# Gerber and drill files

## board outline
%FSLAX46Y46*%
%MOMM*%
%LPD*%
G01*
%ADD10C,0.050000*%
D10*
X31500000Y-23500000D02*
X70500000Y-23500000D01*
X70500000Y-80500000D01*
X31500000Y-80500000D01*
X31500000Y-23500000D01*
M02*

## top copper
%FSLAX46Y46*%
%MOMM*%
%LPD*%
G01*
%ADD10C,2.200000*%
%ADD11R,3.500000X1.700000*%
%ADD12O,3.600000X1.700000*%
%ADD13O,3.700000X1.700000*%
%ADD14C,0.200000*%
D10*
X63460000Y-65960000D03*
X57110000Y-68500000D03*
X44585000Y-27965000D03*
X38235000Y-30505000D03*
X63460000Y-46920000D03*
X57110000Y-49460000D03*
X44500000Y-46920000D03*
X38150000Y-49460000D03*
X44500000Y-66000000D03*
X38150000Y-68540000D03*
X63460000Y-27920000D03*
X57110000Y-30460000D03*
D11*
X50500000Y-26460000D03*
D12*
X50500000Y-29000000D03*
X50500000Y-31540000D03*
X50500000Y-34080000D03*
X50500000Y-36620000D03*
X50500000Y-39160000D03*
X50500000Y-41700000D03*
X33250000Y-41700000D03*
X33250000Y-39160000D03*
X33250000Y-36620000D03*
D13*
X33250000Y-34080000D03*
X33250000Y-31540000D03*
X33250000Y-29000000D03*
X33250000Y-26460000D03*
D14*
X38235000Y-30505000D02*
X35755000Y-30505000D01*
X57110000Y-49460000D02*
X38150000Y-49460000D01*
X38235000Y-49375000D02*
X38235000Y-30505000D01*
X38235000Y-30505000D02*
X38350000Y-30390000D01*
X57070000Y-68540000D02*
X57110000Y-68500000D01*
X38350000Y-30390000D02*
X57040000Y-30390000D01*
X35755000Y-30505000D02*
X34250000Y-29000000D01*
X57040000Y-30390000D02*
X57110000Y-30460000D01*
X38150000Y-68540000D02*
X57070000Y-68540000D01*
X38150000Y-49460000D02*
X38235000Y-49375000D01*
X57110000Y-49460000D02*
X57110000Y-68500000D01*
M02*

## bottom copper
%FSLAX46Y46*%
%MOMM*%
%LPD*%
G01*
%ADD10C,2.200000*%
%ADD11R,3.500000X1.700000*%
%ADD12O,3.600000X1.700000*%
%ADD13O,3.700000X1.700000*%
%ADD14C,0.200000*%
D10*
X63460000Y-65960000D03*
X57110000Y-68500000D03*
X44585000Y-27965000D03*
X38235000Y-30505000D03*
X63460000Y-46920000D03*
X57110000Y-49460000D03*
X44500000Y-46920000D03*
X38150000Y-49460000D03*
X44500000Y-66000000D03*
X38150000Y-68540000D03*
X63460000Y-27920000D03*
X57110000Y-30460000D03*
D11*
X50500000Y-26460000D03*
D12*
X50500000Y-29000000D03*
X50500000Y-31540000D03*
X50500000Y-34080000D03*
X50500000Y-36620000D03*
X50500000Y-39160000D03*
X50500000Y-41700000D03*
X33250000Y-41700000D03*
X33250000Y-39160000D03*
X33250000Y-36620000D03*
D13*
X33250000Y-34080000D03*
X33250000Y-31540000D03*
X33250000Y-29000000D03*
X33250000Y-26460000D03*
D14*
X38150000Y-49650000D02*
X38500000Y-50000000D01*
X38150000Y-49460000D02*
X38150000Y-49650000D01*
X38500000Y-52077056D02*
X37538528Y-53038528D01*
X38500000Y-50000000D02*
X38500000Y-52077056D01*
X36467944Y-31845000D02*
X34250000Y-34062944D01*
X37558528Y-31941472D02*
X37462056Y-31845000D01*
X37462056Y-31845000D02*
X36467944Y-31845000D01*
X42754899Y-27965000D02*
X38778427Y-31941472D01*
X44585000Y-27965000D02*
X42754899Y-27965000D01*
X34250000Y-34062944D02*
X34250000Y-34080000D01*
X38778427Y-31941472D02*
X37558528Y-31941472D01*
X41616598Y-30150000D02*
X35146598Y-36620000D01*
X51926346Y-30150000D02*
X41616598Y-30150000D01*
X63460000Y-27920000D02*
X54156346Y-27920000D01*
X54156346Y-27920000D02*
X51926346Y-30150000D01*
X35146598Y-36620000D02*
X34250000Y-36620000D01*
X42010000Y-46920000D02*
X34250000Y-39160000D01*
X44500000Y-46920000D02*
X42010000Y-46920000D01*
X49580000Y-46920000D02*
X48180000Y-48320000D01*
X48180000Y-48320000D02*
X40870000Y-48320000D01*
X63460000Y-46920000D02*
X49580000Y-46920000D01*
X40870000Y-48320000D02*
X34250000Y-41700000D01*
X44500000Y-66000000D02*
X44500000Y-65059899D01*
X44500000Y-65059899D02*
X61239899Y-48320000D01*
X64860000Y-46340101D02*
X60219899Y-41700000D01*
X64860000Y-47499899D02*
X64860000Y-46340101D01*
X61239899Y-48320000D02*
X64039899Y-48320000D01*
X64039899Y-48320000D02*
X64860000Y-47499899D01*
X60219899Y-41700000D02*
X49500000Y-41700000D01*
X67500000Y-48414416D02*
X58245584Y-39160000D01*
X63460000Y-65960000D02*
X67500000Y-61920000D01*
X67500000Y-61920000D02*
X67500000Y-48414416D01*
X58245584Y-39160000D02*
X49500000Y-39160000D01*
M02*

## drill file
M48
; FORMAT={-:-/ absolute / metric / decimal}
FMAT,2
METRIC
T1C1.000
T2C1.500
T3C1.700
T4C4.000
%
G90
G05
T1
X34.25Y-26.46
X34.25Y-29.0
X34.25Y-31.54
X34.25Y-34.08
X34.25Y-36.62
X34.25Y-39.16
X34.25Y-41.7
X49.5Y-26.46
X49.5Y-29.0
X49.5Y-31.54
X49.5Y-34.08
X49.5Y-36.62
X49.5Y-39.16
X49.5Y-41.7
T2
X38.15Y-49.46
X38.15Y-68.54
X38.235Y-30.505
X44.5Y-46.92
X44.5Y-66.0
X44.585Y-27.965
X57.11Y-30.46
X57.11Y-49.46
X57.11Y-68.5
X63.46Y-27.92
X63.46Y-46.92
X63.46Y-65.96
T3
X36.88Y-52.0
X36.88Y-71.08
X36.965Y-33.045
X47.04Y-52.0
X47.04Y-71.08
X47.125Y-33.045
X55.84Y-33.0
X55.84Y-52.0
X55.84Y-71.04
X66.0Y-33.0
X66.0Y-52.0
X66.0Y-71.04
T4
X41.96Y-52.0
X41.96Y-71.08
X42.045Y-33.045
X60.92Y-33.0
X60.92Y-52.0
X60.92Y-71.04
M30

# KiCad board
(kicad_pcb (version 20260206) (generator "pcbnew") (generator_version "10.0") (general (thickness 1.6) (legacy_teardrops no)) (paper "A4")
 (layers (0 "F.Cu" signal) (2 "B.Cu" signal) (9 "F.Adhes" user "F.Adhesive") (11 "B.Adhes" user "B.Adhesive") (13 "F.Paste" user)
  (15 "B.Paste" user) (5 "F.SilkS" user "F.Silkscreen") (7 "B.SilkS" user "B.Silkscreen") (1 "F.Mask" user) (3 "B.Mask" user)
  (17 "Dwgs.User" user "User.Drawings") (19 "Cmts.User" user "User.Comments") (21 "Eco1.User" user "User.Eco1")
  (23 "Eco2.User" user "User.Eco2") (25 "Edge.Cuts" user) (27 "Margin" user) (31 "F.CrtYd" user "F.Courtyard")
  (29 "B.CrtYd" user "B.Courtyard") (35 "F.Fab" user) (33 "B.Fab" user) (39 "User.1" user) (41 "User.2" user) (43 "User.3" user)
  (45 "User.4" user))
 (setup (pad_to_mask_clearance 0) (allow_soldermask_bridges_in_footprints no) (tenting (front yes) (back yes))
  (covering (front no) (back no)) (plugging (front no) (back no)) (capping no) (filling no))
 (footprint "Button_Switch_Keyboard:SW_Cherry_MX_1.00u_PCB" (layer "F.Cu") (at 63.46 65.96)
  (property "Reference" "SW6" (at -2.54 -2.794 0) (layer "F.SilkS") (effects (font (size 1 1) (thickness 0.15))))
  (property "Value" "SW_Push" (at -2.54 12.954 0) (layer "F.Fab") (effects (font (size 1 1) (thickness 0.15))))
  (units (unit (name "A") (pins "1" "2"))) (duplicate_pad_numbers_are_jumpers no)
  (pad "" np_thru_hole circle (at -7.62 5.08) (size 1.7 1.7) (drill 1.7) (layers "*.Cu" "*.Mask"))
  (pad "" np_thru_hole circle (at -2.54 5.08) (size 4 4) (drill 4) (layers "*.Cu" "*.Mask"))
  (pad "" np_thru_hole circle (at 2.54 5.08) (size 1.7 1.7) (drill 1.7) (layers "*.Cu" "*.Mask"))
  (pad "1" thru_hole circle (at 0 0) (size 2.2 2.2) (drill 1.5) (layers "*.Cu" "*.Mask") (remove_unused_layers no)
   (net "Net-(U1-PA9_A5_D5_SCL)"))
  (pad "2" thru_hole circle (at -6.35 2.54) (size 2.2 2.2) (drill 1.5) (layers "*.Cu" "*.Mask") (remove_unused_layers no) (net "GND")))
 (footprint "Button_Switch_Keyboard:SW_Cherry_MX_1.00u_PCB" (layer "F.Cu") (at 44.585 27.965)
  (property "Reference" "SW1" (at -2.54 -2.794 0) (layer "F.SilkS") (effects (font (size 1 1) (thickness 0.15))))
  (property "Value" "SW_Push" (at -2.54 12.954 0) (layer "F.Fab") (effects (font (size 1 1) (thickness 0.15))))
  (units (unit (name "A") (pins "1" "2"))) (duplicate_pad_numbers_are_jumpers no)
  (pad "" np_thru_hole circle (at -7.62 5.08) (size 1.7 1.7) (drill 1.7) (layers "*.Cu" "*.Mask"))
  (pad "" np_thru_hole circle (at -2.54 5.08) (size 4 4) (drill 4) (layers "*.Cu" "*.Mask"))
  (pad "" np_thru_hole circle (at 2.54 5.08) (size 1.7 1.7) (drill 1.7) (layers "*.Cu" "*.Mask"))
  (pad "1" thru_hole circle (at 0 0) (size 2.2 2.2) (drill 1.5) (layers "*.Cu" "*.Mask") (remove_unused_layers no)
   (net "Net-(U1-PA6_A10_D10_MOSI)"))
  (pad "2" thru_hole circle (at -6.35 2.54) (size 2.2 2.2) (drill 1.5) (layers "*.Cu" "*.Mask") (remove_unused_layers no) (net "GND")))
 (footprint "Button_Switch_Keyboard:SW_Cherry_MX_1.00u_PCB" (layer "F.Cu") (at 63.46 46.92)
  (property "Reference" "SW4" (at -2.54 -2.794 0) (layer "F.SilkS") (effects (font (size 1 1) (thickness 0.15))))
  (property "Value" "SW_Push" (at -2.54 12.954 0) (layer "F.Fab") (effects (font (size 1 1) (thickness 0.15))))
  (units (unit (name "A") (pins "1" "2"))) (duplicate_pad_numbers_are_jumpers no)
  (pad "" np_thru_hole circle (at -7.62 5.08) (size 1.7 1.7) (drill 1.7) (layers "*.Cu" "*.Mask"))
  (pad "" np_thru_hole circle (at -2.54 5.08) (size 4 4) (drill 4) (layers "*.Cu" "*.Mask"))
  (pad "" np_thru_hole circle (at 2.54 5.08) (size 1.7 1.7) (drill 1.7) (layers "*.Cu" "*.Mask"))
  (pad "1" thru_hole circle (at 0 0) (size 2.2 2.2) (drill 1.5) (layers "*.Cu" "*.Mask") (remove_unused_layers no)
   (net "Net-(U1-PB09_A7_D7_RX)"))
  (pad "2" thru_hole circle (at -6.35 2.54) (size 2.2 2.2) (drill 1.5) (layers "*.Cu" "*.Mask") (remove_unused_layers no) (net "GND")))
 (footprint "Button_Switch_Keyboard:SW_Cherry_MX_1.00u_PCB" (layer "F.Cu") (at 44.5 46.92)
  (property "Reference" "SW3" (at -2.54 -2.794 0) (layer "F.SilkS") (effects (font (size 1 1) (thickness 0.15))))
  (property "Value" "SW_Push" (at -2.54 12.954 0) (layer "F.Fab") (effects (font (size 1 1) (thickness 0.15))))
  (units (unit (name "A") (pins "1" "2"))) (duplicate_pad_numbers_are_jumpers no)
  (pad "" np_thru_hole circle (at -7.62 5.08) (size 1.7 1.7) (drill 1.7) (layers "*.Cu" "*.Mask"))
  (pad "" np_thru_hole circle (at -2.54 5.08) (size 4 4) (drill 4) (layers "*.Cu" "*.Mask"))
  (pad "" np_thru_hole circle (at 2.54 5.08) (size 1.7 1.7) (drill 1.7) (layers "*.Cu" "*.Mask"))
  (pad "1" thru_hole circle (at 0 0) (size 2.2 2.2) (drill 1.5) (layers "*.Cu" "*.Mask") (remove_unused_layers no)
   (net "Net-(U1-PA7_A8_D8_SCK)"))
  (pad "2" thru_hole circle (at -6.35 2.54) (size 2.2 2.2) (drill 1.5) (layers "*.Cu" "*.Mask") (remove_unused_layers no) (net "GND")))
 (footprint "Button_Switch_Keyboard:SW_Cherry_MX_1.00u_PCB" (layer "F.Cu") (at 44.5 66)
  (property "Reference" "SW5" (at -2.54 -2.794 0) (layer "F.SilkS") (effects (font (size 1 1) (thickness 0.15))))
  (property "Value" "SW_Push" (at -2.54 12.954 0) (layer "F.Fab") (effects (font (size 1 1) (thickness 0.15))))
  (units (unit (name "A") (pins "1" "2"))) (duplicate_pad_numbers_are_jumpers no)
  (pad "" np_thru_hole circle (at -7.62 5.08) (size 1.7 1.7) (drill 1.7) (layers "*.Cu" "*.Mask"))
  (pad "" np_thru_hole circle (at -2.54 5.08) (size 4 4) (drill 4) (layers "*.Cu" "*.Mask"))
  (pad "" np_thru_hole circle (at 2.54 5.08) (size 1.7 1.7) (drill 1.7) (layers "*.Cu" "*.Mask"))
  (pad "1" thru_hole circle (at 0 0) (size 2.2 2.2) (drill 1.5) (layers "*.Cu" "*.Mask") (remove_unused_layers no)
   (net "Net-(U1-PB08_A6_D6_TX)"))
  (pad "2" thru_hole circle (at -6.35 2.54) (size 2.2 2.2) (drill 1.5) (layers "*.Cu" "*.Mask") (remove_unused_layers no) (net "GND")))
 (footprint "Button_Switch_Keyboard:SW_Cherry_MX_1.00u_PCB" (layer "F.Cu") (at 63.46 27.92)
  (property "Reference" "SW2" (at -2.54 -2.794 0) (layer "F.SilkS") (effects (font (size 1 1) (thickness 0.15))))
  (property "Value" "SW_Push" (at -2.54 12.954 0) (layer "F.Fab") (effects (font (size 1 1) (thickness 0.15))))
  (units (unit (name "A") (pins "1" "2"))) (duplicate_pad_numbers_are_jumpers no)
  (pad "" np_thru_hole circle (at -7.62 5.08) (size 1.7 1.7) (drill 1.7) (layers "*.Cu" "*.Mask"))
  (pad "" np_thru_hole circle (at -2.54 5.08) (size 4 4) (drill 4) (layers "*.Cu" "*.Mask"))
  (pad "" np_thru_hole circle (at 2.54 5.08) (size 1.7 1.7) (drill 1.7) (layers "*.Cu" "*.Mask"))
  (pad "1" thru_hole circle (at 0 0) (size 2.2 2.2) (drill 1.5) (layers "*.Cu" "*.Mask") (remove_unused_layers no)
   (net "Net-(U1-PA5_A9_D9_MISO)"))
  (pad "2" thru_hole circle (at -6.35 2.54) (size 2.2 2.2) (drill 1.5) (layers "*.Cu" "*.Mask") (remove_unused_layers no) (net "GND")))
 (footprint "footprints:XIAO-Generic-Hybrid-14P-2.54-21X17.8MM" (layer "B.Cu") (at 41.875 34.08 180)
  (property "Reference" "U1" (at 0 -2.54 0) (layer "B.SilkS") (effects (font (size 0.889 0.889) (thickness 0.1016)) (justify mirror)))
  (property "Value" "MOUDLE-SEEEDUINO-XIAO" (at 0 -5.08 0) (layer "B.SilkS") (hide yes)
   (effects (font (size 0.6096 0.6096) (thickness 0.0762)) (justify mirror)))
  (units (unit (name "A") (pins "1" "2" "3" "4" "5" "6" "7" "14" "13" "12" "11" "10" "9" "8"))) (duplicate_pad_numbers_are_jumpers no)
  (pad "1" thru_hole rect (at -7.625 7.62 180) (size 3.5 1.7) (drill 1 (offset -1 0)) (layers "*.Cu" "*.Mask") (remove_unused_layers no)
   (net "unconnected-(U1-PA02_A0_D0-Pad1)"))
  (pad "2" thru_hole oval (at -7.625 5.08 180) (size 3.6 1.7) (drill 1 (offset -1 0)) (layers "*.Cu" "*.Mask") (remove_unused_layers no)
   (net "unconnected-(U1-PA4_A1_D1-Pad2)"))
  (pad "3" thru_hole oval (at -7.625 2.54 180) (size 3.6 1.7) (drill 1 (offset -1 0)) (layers "*.Cu" "*.Mask") (remove_unused_layers no)
   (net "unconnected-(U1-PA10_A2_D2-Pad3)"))
  (pad "4" thru_hole oval (at -7.625 0 180) (size 3.6 1.7) (drill 1 (offset -1 0)) (layers "*.Cu" "*.Mask") (remove_unused_layers no)
   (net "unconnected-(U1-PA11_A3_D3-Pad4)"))
  (pad "5" thru_hole oval (at -7.625 -2.54 180) (size 3.6 1.7) (drill 1 (offset -1 0)) (layers "*.Cu" "*.Mask") (remove_unused_layers no)
   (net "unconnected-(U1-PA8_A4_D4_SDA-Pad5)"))
  (pad "6" thru_hole oval (at -7.625 -5.08) (size 3.6 1.7) (drill 1 (offset 1 0)) (layers "*.Cu" "*.Mask") (remove_unused_layers no)
   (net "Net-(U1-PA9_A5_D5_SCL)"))
  (pad "7" thru_hole oval (at -7.625 -7.62 180) (size 3.6 1.7) (drill 1 (offset -1 0)) (layers "*.Cu" "*.Mask") (remove_unused_layers no)
   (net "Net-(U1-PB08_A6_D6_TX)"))
  (pad "8" thru_hole oval (at 7.625 -7.62 180) (size 3.6 1.7) (drill 1 (offset 1 0)) (layers "*.Cu" "*.Mask") (remove_unused_layers no)
   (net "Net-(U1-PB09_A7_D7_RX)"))
  (pad "9" thru_hole oval (at 7.625 -5.08 180) (size 3.6 1.7) (drill 1 (offset 1 0)) (layers "*.Cu" "*.Mask") (remove_unused_layers no)
   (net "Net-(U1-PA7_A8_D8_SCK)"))
  (pad "10" thru_hole oval (at 7.625 -2.54 180) (size 3.6 1.7) (drill 1 (offset 1 0)) (layers "*.Cu" "*.Mask") (remove_unused_layers no)
   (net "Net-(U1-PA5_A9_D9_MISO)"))
  (pad "11" thru_hole oval (at 7.625 0 180) (size 3.7 1.7) (drill 1 (offset 1 0)) (layers "*.Cu" "*.Mask") (remove_unused_layers no)
   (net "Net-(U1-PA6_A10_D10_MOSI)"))
  (pad "12" thru_hole oval (at 7.625 2.54 180) (size 3.7 1.7) (drill 1 (offset 1 0)) (layers "*.Cu" "*.Mask") (remove_unused_layers no)
   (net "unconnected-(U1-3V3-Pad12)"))
  (pad "13" thru_hole oval (at 7.625 5.08 180) (size 3.7 1.7) (drill 1 (offset 1 0)) (layers "*.Cu" "*.Mask") (remove_unused_layers no)
   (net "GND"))
  (pad "14" thru_hole oval (at 7.625 7.62 180) (size 3.7 1.7) (drill 1 (offset 1 0)) (layers "*.Cu" "*.Mask") (remove_unused_layers no)
   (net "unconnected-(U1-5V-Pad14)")))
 (gr_rect (start 31.5 23.5) (end 70.5 80.5) (stroke (width 0.05) (type default)) (fill no) (layer "Edge.Cuts"))
 (segment (start 38.235 30.505) (end 35.755 30.505) (width 0.2) (layer "F.Cu") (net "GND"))
 (segment (start 57.11 49.46) (end 38.15 49.46) (width 0.2) (layer "F.Cu") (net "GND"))
 (segment (start 38.235 49.375) (end 38.235 30.505) (width 0.2) (layer "F.Cu") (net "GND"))
 (segment (start 38.235 30.505) (end 38.35 30.39) (width 0.2) (layer "F.Cu") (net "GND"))
 (segment (start 57.07 68.54) (end 57.11 68.5) (width 0.2) (layer "F.Cu") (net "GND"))
 (segment (start 38.35 30.39) (end 57.04 30.39) (width 0.2) (layer "F.Cu") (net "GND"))
 (segment (start 35.755 30.505) (end 34.25 29) (width 0.2) (layer "F.Cu") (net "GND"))
 (segment (start 57.04 30.39) (end 57.11 30.46) (width 0.2) (layer "F.Cu") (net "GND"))
 (segment (start 38.15 68.54) (end 57.07 68.54) (width 0.2) (layer "F.Cu") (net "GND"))
 (segment (start 38.15 49.46) (end 38.235 49.375) (width 0.2) (layer "F.Cu") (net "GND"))
 (segment (start 57.11 49.46) (end 57.11 68.5) (width 0.2) (layer "F.Cu") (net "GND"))
 (segment (start 38.15 49.65) (end 38.5 50) (width 0.2) (layer "B.Cu") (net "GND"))
 (segment (start 38.15 49.46) (end 38.15 49.65) (width 0.2) (layer "B.Cu") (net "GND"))
 (segment (start 38.5 52.077056) (end 37.538528 53.038528) (width 0.2) (layer "B.Cu") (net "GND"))
 (segment (start 38.5 50) (end 38.5 52.077056) (width 0.2) (layer "B.Cu") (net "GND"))
 (segment (start 36.467944 31.845) (end 34.25 34.062944) (width 0.2) (layer "B.Cu") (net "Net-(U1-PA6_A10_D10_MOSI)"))
 (segment (start 37.558528 31.941472) (end 37.462056 31.845) (width 0.2) (layer "B.Cu") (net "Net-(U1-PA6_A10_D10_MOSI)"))
 (segment (start 37.462056 31.845) (end 36.467944 31.845) (width 0.2) (layer "B.Cu") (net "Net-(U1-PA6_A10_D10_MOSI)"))
 (segment (start 42.754899 27.965) (end 38.778427 31.941472) (width 0.2) (layer "B.Cu") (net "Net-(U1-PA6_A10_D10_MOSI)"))
 (segment (start 44.585 27.965) (end 42.754899 27.965) (width 0.2) (layer "B.Cu") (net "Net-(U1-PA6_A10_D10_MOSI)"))
 (segment (start 34.25 34.062944) (end 34.25 34.08) (width 0.2) (layer "B.Cu") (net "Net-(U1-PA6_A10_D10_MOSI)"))
 (segment (start 38.778427 31.941472) (end 37.558528 31.941472) (width 0.2) (layer "B.Cu") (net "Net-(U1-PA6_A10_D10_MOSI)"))
 (segment (start 41.616598 30.15) (end 35.146598 36.62) (width 0.2) (layer "B.Cu") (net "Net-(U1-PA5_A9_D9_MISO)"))
 (segment (start 51.926346 30.15) (end 41.616598 30.15) (width 0.2) (layer "B.Cu") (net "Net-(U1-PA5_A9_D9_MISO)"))
 (segment (start 63.46 27.92) (end 54.156346 27.92) (width 0.2) (layer "B.Cu") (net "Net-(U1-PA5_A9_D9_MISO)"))
 (segment (start 54.156346 27.92) (end 51.926346 30.15) (width 0.2) (layer "B.Cu") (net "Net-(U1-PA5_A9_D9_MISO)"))
 (segment (start 35.146598 36.62) (end 34.25 36.62) (width 0.2) (layer "B.Cu") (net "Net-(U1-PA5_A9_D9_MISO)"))
 (segment (start 42.01 46.92) (end 34.25 39.16) (width 0.2) (layer "B.Cu") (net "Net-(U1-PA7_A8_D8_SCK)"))
 (segment (start 44.5 46.92) (end 42.01 46.92) (width 0.2) (layer "B.Cu") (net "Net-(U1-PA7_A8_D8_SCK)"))
 (segment (start 49.58 46.92) (end 48.18 48.32) (width 0.2) (layer "B.Cu") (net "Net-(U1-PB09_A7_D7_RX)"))
 (segment (start 48.18 48.32) (end 40.87 48.32) (width 0.2) (layer "B.Cu") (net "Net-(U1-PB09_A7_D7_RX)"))
 (segment (start 63.46 46.92) (end 49.58 46.92) (width 0.2) (layer "B.Cu") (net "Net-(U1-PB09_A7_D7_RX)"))
 (segment (start 40.87 48.32) (end 34.25 41.7) (width 0.2) (layer "B.Cu") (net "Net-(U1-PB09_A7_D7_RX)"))
 (segment (start 44.5 66) (end 44.5 65.059899) (width 0.2) (layer "B.Cu") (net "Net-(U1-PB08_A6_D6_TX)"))
 (segment (start 44.5 65.059899) (end 61.239899 48.32) (width 0.2) (layer "B.Cu") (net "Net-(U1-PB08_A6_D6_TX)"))
 (segment (start 64.86 46.340101) (end 60.219899 41.7) (width 0.2) (layer "B.Cu") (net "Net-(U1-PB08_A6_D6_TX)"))
 (segment (start 64.86 47.499899) (end 64.86 46.340101) (width 0.2) (layer "B.Cu") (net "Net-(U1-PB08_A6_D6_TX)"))
 (segment (start 61.239899 48.32) (end 64.039899 48.32) (width 0.2) (layer "B.Cu") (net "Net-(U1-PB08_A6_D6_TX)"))
 (segment (start 64.039899 48.32) (end 64.86 47.499899) (width 0.2) (layer "B.Cu") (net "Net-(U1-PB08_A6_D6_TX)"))
 (segment (start 60.219899 41.7) (end 49.5 41.7) (width 0.2) (layer "B.Cu") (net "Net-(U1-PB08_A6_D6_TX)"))
 (segment (start 67.5 48.414416) (end 58.245584 39.16) (width 0.2) (layer "B.Cu") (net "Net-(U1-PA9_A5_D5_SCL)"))
 (segment (start 63.46 65.96) (end 67.5 61.92) (width 0.2) (layer "B.Cu") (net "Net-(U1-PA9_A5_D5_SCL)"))
 (segment (start 67.5 61.92) (end 67.5 48.414416) (width 0.2) (layer "B.Cu") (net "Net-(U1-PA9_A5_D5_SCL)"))
 (segment (start 58.245584 39.16) (end 49.5 39.16) (width 0.2) (layer "B.Cu") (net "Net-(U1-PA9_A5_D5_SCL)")))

